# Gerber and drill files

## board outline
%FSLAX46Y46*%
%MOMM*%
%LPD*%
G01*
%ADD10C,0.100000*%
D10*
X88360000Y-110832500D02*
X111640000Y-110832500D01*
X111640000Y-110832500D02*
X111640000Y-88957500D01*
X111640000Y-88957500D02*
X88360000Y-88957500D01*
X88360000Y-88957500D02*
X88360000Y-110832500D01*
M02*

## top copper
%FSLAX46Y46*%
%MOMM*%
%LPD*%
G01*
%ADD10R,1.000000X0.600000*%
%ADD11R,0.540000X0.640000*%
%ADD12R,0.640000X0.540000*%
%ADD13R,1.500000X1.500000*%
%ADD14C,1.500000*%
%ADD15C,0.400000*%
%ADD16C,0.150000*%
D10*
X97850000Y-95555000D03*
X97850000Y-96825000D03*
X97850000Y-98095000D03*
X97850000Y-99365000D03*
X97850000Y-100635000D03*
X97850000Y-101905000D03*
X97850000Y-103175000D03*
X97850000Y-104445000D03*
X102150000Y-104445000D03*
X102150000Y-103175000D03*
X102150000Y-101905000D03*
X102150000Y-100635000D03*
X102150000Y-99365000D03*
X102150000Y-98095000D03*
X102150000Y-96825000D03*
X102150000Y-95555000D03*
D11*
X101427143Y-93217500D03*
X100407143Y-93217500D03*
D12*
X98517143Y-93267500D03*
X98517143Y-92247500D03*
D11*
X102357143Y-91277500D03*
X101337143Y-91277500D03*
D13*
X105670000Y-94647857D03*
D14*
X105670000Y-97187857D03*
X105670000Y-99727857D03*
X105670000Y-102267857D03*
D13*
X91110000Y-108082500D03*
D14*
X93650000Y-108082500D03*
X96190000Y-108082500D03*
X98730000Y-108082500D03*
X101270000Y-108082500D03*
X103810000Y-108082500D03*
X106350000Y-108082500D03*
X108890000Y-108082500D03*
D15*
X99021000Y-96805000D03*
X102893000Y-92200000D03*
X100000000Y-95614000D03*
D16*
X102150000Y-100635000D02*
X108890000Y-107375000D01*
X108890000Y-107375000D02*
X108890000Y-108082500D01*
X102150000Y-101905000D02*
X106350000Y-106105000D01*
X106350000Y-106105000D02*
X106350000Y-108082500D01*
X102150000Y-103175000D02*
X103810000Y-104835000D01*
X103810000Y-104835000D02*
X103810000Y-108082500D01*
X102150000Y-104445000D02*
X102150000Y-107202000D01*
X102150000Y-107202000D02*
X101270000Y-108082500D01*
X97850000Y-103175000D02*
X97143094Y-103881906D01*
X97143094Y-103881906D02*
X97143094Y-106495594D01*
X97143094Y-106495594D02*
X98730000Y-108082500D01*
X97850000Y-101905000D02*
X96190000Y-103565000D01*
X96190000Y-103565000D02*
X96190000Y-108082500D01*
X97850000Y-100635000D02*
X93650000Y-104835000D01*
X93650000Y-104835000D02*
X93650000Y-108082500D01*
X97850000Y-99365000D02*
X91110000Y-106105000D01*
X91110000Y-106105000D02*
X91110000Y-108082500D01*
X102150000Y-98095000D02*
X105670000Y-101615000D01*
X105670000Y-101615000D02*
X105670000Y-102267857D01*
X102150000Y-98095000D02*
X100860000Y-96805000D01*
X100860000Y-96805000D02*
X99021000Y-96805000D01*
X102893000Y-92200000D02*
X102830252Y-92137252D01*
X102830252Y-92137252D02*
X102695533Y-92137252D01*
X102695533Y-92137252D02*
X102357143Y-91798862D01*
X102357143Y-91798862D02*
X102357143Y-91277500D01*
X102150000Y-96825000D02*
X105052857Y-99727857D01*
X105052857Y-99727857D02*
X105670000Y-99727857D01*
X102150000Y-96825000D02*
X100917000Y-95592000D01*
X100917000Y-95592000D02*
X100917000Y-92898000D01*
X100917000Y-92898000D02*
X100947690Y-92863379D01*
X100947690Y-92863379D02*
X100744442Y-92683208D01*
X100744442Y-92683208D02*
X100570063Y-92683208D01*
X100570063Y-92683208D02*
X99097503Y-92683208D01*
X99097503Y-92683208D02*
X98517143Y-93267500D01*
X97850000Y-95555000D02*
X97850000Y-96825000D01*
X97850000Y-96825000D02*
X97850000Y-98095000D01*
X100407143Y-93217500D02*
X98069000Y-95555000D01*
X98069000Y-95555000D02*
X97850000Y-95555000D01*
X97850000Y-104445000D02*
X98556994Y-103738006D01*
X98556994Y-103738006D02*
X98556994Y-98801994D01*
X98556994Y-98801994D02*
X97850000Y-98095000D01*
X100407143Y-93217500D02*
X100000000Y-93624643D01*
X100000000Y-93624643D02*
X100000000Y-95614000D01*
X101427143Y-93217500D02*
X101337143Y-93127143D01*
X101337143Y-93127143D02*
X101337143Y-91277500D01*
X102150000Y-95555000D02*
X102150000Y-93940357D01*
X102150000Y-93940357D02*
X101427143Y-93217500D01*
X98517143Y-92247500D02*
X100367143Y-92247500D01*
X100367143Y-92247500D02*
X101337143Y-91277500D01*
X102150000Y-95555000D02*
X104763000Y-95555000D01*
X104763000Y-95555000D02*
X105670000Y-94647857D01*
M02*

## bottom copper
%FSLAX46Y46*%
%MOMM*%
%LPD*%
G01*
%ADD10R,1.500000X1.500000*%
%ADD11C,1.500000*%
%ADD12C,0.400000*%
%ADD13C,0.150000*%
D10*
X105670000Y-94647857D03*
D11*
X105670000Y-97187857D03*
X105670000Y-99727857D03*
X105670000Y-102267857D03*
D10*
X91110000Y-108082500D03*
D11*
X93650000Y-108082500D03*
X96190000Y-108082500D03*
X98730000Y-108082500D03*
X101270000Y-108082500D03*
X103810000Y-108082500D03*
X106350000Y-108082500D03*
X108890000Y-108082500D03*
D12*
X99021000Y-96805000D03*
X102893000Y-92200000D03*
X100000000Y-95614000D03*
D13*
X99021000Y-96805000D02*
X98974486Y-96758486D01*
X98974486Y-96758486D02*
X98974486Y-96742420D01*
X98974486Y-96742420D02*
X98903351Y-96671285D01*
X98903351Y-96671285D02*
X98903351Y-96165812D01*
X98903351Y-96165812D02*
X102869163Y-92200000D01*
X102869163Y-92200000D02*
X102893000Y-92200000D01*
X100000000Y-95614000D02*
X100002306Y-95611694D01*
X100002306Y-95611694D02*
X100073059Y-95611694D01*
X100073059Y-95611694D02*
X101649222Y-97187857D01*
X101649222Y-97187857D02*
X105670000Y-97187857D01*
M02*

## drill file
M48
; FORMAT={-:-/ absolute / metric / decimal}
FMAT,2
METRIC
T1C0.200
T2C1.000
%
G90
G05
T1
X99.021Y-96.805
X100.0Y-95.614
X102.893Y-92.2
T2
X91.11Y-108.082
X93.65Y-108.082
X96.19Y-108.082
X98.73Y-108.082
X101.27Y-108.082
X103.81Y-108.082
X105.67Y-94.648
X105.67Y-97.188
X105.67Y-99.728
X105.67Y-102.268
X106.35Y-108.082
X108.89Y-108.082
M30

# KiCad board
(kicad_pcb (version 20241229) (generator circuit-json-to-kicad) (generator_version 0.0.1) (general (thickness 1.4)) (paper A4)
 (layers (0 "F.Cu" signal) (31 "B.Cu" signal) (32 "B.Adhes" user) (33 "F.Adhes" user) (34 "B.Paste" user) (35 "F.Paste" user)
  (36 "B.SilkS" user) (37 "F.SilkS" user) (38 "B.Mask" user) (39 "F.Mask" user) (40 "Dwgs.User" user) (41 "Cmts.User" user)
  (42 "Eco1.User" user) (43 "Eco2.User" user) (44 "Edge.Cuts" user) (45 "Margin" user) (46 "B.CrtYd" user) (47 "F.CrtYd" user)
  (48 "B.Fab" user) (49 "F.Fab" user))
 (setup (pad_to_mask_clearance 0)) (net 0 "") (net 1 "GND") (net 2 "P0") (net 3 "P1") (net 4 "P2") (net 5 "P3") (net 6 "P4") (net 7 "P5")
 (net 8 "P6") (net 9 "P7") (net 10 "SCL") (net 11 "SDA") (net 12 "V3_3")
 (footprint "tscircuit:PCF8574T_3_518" (layer F.Cu) (at 100 100 0)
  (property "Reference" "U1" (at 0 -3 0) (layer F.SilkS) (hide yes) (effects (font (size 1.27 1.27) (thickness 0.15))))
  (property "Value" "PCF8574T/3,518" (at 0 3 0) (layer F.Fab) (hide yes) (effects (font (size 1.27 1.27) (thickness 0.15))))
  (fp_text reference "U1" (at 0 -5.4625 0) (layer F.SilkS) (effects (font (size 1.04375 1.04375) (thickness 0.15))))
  (pad "1" smd rect (at -2.15 -4.445 0) (size 1 0.6) (layers F.Cu F.Paste F.Mask) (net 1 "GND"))
  (pad "2" smd rect (at -2.15 -3.1750000000000003 0) (size 1 0.6) (layers F.Cu F.Paste F.Mask) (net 1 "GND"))
  (pad "3" smd rect (at -2.15 -1.9050000000000002 0) (size 1 0.6) (layers F.Cu F.Paste F.Mask) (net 1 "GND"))
  (pad "4" smd rect (at -2.15 -0.6350000000000002 0) (size 1 0.6) (layers F.Cu F.Paste F.Mask) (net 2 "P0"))
  (pad "5" smd rect (at -2.15 0.6349999999999998 0) (size 1 0.6) (layers F.Cu F.Paste F.Mask) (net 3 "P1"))
  (pad "6" smd rect (at -2.15 1.9049999999999994 0) (size 1 0.6) (layers F.Cu F.Paste F.Mask) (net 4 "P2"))
  (pad "7" smd rect (at -2.15 3.175 0) (size 1 0.6) (layers F.Cu F.Paste F.Mask) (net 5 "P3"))
  (pad "8" smd rect (at -2.15 4.445 0) (size 1 0.6) (layers F.Cu F.Paste F.Mask) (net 1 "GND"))
  (pad "9" smd rect (at 2.15 4.445 0) (size 1 0.6) (layers F.Cu F.Paste F.Mask) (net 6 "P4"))
  (pad "10" smd rect (at 2.15 3.1750000000000003 0) (size 1 0.6) (layers F.Cu F.Paste F.Mask) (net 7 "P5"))
  (pad "11" smd rect (at 2.15 1.9050000000000002 0) (size 1 0.6) (layers F.Cu F.Paste F.Mask) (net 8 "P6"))
  (pad "12" smd rect (at 2.15 0.6350000000000002 0) (size 1 0.6) (layers F.Cu F.Paste F.Mask) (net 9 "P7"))
  (pad "13" smd rect (at 2.15 -0.6349999999999998 0) (size 1 0.6) (layers F.Cu F.Paste F.Mask))
  (pad "14" smd rect (at 2.15 -1.9049999999999994 0) (size 1 0.6) (layers F.Cu F.Paste F.Mask) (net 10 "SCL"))
  (pad "15" smd rect (at 2.15 -3.175 0) (size 1 0.6) (layers F.Cu F.Paste F.Mask) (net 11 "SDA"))
  (pad "16" smd rect (at 2.15 -4.445 0) (size 1 0.6) (layers F.Cu F.Paste F.Mask) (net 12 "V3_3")))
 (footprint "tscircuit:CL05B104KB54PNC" (layer F.Cu) (at 100.91714285714286 93.2175 180)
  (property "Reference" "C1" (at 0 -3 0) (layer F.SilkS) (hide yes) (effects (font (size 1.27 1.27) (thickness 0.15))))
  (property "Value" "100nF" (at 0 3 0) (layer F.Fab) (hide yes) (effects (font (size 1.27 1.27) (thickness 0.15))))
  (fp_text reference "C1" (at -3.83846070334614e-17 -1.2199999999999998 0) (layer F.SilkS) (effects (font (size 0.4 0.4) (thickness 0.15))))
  (pad "1" smd rect (at -0.5099999999999999 0 0) (size 0.54 0.64) (layers F.Cu F.Paste F.Mask) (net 12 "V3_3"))
  (pad "2" smd rect (at 0.51 0 0) (size 0.54 0.64) (layers F.Cu F.Paste F.Mask) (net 1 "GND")))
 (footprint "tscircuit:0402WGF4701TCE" (layer F.Cu) (at 98.51714285714286 92.7575 90)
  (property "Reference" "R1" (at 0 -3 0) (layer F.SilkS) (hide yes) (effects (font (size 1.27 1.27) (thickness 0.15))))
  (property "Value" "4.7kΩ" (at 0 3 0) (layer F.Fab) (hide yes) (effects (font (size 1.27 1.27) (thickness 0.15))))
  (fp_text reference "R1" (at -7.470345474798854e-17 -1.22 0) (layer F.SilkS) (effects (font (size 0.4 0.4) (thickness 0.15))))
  (pad "1" smd rect (at -0.5099999999999998 0 0) (size 0.64 0.54) (layers F.Cu F.Paste F.Mask) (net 11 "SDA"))
  (pad "2" smd rect (at 0.5099999999999998 0 0) (size 0.64 0.54) (layers F.Cu F.Paste F.Mask) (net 12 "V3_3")))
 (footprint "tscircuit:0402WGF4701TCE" (layer F.Cu) (at 101.84714285714286 91.2775 180)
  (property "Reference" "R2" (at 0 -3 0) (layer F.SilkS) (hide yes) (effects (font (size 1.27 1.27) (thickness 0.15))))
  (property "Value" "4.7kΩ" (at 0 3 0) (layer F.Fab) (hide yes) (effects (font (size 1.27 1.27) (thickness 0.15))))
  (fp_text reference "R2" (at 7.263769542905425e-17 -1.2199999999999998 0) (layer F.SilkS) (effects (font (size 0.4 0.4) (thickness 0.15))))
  (pad "1" smd rect (at -0.51 0 0) (size 0.54 0.64) (layers F.Cu F.Paste F.Mask) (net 10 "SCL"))
  (pad "2" smd rect (at 0.51 0 0) (size 0.54 0.64) (layers F.Cu F.Paste F.Mask) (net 12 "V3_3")))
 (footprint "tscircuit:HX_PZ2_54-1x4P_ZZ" (layer F.Cu) (at 105.67 98.45785714285714 -90.00000000000001)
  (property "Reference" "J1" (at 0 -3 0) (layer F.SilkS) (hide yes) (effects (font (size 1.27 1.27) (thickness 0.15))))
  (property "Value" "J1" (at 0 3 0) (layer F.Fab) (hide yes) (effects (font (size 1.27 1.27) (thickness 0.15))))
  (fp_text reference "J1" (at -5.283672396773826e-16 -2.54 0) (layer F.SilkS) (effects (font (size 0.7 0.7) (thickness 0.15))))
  (pad "1" thru_hole rect (at -3.81 5.705062545910424e-16 0) (size 1.5 1.5) (drill 1) (layers *.Cu *.Mask) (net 12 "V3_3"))
  (pad "2" thru_hole circle (at -1.27 4.862282247637226e-16 0) (size 1.5 1.5) (drill 1) (layers *.Cu *.Mask) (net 1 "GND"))
  (pad "3" thru_hole circle (at 1.27 -4.862282247637226e-16 0) (size 1.5 1.5) (drill 1) (layers *.Cu *.Mask) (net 11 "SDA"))
  (pad "4" thru_hole circle (at 3.81 -5.705062545910424e-16 0) (size 1.5 1.5) (drill 1) (layers *.Cu *.Mask) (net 10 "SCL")))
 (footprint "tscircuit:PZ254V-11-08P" (layer F.Cu) (at 100 108.0825 0)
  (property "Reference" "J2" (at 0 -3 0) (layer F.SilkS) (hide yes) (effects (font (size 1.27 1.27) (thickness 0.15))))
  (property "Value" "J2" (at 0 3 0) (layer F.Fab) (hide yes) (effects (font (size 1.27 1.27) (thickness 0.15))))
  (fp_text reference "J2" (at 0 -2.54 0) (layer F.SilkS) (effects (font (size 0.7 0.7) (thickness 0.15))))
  (pad "1" thru_hole rect (at -8.89 0 0) (size 1.5 1.5) (drill 1) (layers *.Cu *.Mask) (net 2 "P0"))
  (pad "2" thru_hole circle (at -6.3500000000000005 0 0) (size 1.5 1.5) (drill 1) (layers *.Cu *.Mask) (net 3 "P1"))
  (pad "3" thru_hole circle (at -3.8100000000000005 0 0) (size 1.5 1.5) (drill 1) (layers *.Cu *.Mask) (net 4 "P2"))
  (pad "4" thru_hole circle (at -1.2700000000000005 0 0) (size 1.5 1.5) (drill 1) (layers *.Cu *.Mask) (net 5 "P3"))
  (pad "5" thru_hole circle (at 1.2699999999999996 0 0) (size 1.5 1.5) (drill 1) (layers *.Cu *.Mask) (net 6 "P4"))
  (pad "6" thru_hole circle (at 3.8099999999999987 0 0) (size 1.5 1.5) (drill 1) (layers *.Cu *.Mask) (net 7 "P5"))
  (pad "7" thru_hole circle (at 6.35 0 0) (size 1.5 1.5) (drill 1) (layers *.Cu *.Mask) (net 8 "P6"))
  (pad "8" thru_hole circle (at 8.89 0 0) (size 1.5 1.5) (drill 1) (layers *.Cu *.Mask) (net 9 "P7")))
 (segment (start 102.15 100.635) (end 108.89 107.375) (width 0.15) (layer F.Cu) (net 9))
 (segment (start 108.89 107.375) (end 108.89 108.0825) (width 0.15) (layer F.Cu) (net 9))
 (segment (start 102.15 101.905) (end 106.35 106.105) (width 0.15) (layer F.Cu) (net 8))
 (segment (start 106.35 106.105) (end 106.35 108.0825) (width 0.15) (layer F.Cu) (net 8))
 (segment (start 102.15 103.175) (end 103.81 104.835) (width 0.15) (layer F.Cu) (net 7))
 (segment (start 103.81 104.835) (end 103.81 108.0825) (width 0.15) (layer F.Cu) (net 7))
 (segment (start 102.15 104.445) (end 102.15 107.202) (width 0.15) (layer F.Cu) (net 6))
 (segment (start 102.15 107.202) (end 101.27 108.0825) (width 0.15) (layer F.Cu) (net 6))
 (segment (start 97.85 103.175) (end 97.14309387785406 103.88190612214595) (width 0.15) (layer F.Cu) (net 5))
 (segment (start 97.14309387785406 103.88190612214595) (end 97.14309387785406 106.49559387785405) (width 0.15) (layer F.Cu) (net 5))
 (segment (start 97.14309387785406 106.49559387785405) (end 98.73 108.0825) (width 0.15) (layer F.Cu) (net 5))
 (segment (start 97.85 101.905) (end 96.19 103.565) (width 0.15) (layer F.Cu) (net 4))
 (segment (start 96.19 103.565) (end 96.19 108.0825) (width 0.15) (layer F.Cu) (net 4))
 (segment (start 97.85 100.635) (end 93.65 104.83500000000001) (width 0.15) (layer F.Cu) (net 3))
 (segment (start 93.65 104.83500000000001) (end 93.65 108.0825) (width 0.15) (layer F.Cu) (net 3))
 (segment (start 97.85 99.365) (end 91.11 106.105) (width 0.15) (layer F.Cu) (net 2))
 (segment (start 91.11 106.105) (end 91.11 108.0825) (width 0.15) (layer F.Cu) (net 2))
 (segment (start 102.15 98.095) (end 105.67 101.615) (width 0.15) (layer F.Cu) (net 10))
 (segment (start 105.67 101.615) (end 105.67 102.26785714285714) (width 0.15) (layer F.Cu) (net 10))
 (segment (start 102.15 98.095) (end 100.86 96.805) (width 0.15) (layer F.Cu) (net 10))
 (segment (start 100.86 96.805) (end 99.021 96.805) (width 0.15) (layer F.Cu) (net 10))
 (segment (start 99.021 96.805) (end 98.97448570689265 96.75848570689264) (width 0.15) (layer B.Cu) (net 10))
 (segment (start 98.97448570689265 96.75848570689264) (end 98.97448570689265 96.7424195752621) (width 0.15) (layer B.Cu) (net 10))
 (segment (start 98.97448570689265 96.7424195752621) (end 98.90335073935582 96.67128460772527) (width 0.15) (layer B.Cu) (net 10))
 (segment (start 98.90335073935582 96.67128460772527) (end 98.90335073935582 96.1658122704005) (width 0.15) (layer B.Cu) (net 10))
 (segment (start 98.90335073935582 96.1658122704005) (end 102.86916300975629 92.2) (width 0.15) (layer B.Cu) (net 10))
 (segment (start 102.86916300975629 92.2) (end 102.893 92.2) (width 0.15) (layer B.Cu) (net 10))
 (segment (start 102.893 92.2) (end 102.83025181571226 92.13725181571226) (width 0.15) (layer F.Cu) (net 10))
 (segment (start 102.83025181571226 92.13725181571226) (end 102.69553276752963 92.13725181571226) (width 0.15) (layer F.Cu) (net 10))
 (segment (start 102.69553276752963 92.13725181571226) (end 102.35714285714286 91.7988619053255) (width 0.15) (layer F.Cu) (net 10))
 (segment (start 102.35714285714286 91.7988619053255) (end 102.35714285714286 91.2775) (width 0.15) (layer F.Cu) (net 10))
 (segment (start 102.15 96.825) (end 105.05285714285714 99.72785714285715) (width 0.15) (layer F.Cu) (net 11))
 (segment (start 105.05285714285714 99.72785714285715) (end 105.67 99.72785714285715) (width 0.15) (layer F.Cu) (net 11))
 (segment (start 102.15 96.825) (end 100.917 95.592) (width 0.15) (layer F.Cu) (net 11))
 (segment (start 100.917 95.592) (end 100.917 92.898) (width 0.15) (layer F.Cu) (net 11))
 (segment (start 100.917 92.898) (end 100.9476902638268 92.8633786928267) (width 0.15) (layer F.Cu) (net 11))
 (segment (start 100.9476902638268 92.8633786928267) (end 100.7444423942015 92.68320840896624) (width 0.15) (layer F.Cu) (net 11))
 (segment (start 100.7444423942015 92.68320840896624) (end 100.57006282266266 92.68320840896624) (width 0.15) (layer F.Cu) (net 11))
 (segment (start 100.57006282266266 92.68320840896624) (end 99.09750340483012 92.68320840896624) (width 0.15) (layer F.Cu) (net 11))
 (segment (start 99.09750340483012 92.68320840896624) (end 98.51714285714286 93.2675) (width 0.15) (layer F.Cu) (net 11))
 (segment (start 97.85 95.555) (end 97.85 96.825) (width 0.15) (layer F.Cu) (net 1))
 (segment (start 97.85 96.825) (end 97.85 98.095) (width 0.15) (layer F.Cu) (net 1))
 (segment (start 100.40714285714286 93.2175) (end 98.069 95.555) (width 0.15) (layer F.Cu) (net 1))
 (segment (start 98.069 95.555) (end 97.85 95.555) (width 0.15) (layer F.Cu) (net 1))
 (segment (start 97.85 104.445) (end 98.55699418028716 103.73800581971284) (width 0.15) (layer F.Cu) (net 1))
 (segment (start 98.55699418028716 103.73800581971284) (end 98.55699418028716 98.80199418028717) (width 0.15) (layer F.Cu) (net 1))
 (segment (start 98.55699418028716 98.80199418028717) (end 97.85 98.095) (width 0.15) (layer F.Cu) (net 1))
 (segment (start 100.40714285714286 93.2175) (end 100 93.62464285714286) (width 0.15) (layer F.Cu) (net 1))
 (segment (start 100 93.62464285714286) (end 100 95.614) (width 0.15) (layer F.Cu) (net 1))
 (segment (start 100 95.614) (end 100.0023057762355 95.6116942237645) (width 0.15) (layer B.Cu) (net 1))
 (segment (start 100.0023057762355 95.6116942237645) (end 100.07305874681478 95.6116942237645) (width 0.15) (layer B.Cu) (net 1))
 (segment (start 100.07305874681478 95.6116942237645) (end 101.64922166590743 97.18785714285714) (width 0.15) (layer B.Cu) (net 1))
 (segment (start 101.64922166590743 97.18785714285714) (end 105.67 97.18785714285714) (width 0.15) (layer B.Cu) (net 1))
 (segment (start 101.42714285714285 93.2175) (end 101.33714285714285 93.12714285714286) (width 0.15) (layer F.Cu) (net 12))
 (segment (start 101.33714285714285 93.12714285714286) (end 101.33714285714285 91.2775) (width 0.15) (layer F.Cu) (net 12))
 (segment (start 102.15 95.555) (end 102.15 93.94035714285714) (width 0.15) (layer F.Cu) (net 12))
 (segment (start 102.15 93.94035714285714) (end 101.42714285714285 93.2175) (width 0.15) (layer F.Cu) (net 12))
 (segment (start 98.51714285714286 92.2475) (end 100.36714285714285 92.2475) (width 0.15) (layer F.Cu) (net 12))
 (segment (start 100.36714285714285 92.2475) (end 101.33714285714285 91.2775) (width 0.15) (layer F.Cu) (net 12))
 (segment (start 102.15 95.555) (end 104.763 95.555) (width 0.15) (layer F.Cu) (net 12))
 (segment (start 104.763 95.555) (end 105.67 94.64785714285715) (width 0.15) (layer F.Cu) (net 12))
 (gr_line (start 88.36 110.8325) (end 111.64 110.8325) (width 0.1) (layer Edge.Cuts))
 (gr_line (start 111.64 110.8325) (end 111.64 88.9575) (width 0.1) (layer Edge.Cuts))
 (gr_line (start 111.64 88.9575) (end 88.36 88.9575) (width 0.1) (layer Edge.Cuts))
 (gr_line (start 88.36 88.9575) (end 88.36 110.8325) (width 0.1) (layer Edge.Cuts))
 (via (at 99.021 96.805) (size 0.4) (drill 0.2) (layers F.Cu B.Cu) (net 10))
 (via (at 102.893 92.2) (size 0.4) (drill 0.2) (layers F.Cu B.Cu) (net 10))
 (via (at 100 95.614) (size 0.4) (drill 0.2) (layers F.Cu B.Cu) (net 1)))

